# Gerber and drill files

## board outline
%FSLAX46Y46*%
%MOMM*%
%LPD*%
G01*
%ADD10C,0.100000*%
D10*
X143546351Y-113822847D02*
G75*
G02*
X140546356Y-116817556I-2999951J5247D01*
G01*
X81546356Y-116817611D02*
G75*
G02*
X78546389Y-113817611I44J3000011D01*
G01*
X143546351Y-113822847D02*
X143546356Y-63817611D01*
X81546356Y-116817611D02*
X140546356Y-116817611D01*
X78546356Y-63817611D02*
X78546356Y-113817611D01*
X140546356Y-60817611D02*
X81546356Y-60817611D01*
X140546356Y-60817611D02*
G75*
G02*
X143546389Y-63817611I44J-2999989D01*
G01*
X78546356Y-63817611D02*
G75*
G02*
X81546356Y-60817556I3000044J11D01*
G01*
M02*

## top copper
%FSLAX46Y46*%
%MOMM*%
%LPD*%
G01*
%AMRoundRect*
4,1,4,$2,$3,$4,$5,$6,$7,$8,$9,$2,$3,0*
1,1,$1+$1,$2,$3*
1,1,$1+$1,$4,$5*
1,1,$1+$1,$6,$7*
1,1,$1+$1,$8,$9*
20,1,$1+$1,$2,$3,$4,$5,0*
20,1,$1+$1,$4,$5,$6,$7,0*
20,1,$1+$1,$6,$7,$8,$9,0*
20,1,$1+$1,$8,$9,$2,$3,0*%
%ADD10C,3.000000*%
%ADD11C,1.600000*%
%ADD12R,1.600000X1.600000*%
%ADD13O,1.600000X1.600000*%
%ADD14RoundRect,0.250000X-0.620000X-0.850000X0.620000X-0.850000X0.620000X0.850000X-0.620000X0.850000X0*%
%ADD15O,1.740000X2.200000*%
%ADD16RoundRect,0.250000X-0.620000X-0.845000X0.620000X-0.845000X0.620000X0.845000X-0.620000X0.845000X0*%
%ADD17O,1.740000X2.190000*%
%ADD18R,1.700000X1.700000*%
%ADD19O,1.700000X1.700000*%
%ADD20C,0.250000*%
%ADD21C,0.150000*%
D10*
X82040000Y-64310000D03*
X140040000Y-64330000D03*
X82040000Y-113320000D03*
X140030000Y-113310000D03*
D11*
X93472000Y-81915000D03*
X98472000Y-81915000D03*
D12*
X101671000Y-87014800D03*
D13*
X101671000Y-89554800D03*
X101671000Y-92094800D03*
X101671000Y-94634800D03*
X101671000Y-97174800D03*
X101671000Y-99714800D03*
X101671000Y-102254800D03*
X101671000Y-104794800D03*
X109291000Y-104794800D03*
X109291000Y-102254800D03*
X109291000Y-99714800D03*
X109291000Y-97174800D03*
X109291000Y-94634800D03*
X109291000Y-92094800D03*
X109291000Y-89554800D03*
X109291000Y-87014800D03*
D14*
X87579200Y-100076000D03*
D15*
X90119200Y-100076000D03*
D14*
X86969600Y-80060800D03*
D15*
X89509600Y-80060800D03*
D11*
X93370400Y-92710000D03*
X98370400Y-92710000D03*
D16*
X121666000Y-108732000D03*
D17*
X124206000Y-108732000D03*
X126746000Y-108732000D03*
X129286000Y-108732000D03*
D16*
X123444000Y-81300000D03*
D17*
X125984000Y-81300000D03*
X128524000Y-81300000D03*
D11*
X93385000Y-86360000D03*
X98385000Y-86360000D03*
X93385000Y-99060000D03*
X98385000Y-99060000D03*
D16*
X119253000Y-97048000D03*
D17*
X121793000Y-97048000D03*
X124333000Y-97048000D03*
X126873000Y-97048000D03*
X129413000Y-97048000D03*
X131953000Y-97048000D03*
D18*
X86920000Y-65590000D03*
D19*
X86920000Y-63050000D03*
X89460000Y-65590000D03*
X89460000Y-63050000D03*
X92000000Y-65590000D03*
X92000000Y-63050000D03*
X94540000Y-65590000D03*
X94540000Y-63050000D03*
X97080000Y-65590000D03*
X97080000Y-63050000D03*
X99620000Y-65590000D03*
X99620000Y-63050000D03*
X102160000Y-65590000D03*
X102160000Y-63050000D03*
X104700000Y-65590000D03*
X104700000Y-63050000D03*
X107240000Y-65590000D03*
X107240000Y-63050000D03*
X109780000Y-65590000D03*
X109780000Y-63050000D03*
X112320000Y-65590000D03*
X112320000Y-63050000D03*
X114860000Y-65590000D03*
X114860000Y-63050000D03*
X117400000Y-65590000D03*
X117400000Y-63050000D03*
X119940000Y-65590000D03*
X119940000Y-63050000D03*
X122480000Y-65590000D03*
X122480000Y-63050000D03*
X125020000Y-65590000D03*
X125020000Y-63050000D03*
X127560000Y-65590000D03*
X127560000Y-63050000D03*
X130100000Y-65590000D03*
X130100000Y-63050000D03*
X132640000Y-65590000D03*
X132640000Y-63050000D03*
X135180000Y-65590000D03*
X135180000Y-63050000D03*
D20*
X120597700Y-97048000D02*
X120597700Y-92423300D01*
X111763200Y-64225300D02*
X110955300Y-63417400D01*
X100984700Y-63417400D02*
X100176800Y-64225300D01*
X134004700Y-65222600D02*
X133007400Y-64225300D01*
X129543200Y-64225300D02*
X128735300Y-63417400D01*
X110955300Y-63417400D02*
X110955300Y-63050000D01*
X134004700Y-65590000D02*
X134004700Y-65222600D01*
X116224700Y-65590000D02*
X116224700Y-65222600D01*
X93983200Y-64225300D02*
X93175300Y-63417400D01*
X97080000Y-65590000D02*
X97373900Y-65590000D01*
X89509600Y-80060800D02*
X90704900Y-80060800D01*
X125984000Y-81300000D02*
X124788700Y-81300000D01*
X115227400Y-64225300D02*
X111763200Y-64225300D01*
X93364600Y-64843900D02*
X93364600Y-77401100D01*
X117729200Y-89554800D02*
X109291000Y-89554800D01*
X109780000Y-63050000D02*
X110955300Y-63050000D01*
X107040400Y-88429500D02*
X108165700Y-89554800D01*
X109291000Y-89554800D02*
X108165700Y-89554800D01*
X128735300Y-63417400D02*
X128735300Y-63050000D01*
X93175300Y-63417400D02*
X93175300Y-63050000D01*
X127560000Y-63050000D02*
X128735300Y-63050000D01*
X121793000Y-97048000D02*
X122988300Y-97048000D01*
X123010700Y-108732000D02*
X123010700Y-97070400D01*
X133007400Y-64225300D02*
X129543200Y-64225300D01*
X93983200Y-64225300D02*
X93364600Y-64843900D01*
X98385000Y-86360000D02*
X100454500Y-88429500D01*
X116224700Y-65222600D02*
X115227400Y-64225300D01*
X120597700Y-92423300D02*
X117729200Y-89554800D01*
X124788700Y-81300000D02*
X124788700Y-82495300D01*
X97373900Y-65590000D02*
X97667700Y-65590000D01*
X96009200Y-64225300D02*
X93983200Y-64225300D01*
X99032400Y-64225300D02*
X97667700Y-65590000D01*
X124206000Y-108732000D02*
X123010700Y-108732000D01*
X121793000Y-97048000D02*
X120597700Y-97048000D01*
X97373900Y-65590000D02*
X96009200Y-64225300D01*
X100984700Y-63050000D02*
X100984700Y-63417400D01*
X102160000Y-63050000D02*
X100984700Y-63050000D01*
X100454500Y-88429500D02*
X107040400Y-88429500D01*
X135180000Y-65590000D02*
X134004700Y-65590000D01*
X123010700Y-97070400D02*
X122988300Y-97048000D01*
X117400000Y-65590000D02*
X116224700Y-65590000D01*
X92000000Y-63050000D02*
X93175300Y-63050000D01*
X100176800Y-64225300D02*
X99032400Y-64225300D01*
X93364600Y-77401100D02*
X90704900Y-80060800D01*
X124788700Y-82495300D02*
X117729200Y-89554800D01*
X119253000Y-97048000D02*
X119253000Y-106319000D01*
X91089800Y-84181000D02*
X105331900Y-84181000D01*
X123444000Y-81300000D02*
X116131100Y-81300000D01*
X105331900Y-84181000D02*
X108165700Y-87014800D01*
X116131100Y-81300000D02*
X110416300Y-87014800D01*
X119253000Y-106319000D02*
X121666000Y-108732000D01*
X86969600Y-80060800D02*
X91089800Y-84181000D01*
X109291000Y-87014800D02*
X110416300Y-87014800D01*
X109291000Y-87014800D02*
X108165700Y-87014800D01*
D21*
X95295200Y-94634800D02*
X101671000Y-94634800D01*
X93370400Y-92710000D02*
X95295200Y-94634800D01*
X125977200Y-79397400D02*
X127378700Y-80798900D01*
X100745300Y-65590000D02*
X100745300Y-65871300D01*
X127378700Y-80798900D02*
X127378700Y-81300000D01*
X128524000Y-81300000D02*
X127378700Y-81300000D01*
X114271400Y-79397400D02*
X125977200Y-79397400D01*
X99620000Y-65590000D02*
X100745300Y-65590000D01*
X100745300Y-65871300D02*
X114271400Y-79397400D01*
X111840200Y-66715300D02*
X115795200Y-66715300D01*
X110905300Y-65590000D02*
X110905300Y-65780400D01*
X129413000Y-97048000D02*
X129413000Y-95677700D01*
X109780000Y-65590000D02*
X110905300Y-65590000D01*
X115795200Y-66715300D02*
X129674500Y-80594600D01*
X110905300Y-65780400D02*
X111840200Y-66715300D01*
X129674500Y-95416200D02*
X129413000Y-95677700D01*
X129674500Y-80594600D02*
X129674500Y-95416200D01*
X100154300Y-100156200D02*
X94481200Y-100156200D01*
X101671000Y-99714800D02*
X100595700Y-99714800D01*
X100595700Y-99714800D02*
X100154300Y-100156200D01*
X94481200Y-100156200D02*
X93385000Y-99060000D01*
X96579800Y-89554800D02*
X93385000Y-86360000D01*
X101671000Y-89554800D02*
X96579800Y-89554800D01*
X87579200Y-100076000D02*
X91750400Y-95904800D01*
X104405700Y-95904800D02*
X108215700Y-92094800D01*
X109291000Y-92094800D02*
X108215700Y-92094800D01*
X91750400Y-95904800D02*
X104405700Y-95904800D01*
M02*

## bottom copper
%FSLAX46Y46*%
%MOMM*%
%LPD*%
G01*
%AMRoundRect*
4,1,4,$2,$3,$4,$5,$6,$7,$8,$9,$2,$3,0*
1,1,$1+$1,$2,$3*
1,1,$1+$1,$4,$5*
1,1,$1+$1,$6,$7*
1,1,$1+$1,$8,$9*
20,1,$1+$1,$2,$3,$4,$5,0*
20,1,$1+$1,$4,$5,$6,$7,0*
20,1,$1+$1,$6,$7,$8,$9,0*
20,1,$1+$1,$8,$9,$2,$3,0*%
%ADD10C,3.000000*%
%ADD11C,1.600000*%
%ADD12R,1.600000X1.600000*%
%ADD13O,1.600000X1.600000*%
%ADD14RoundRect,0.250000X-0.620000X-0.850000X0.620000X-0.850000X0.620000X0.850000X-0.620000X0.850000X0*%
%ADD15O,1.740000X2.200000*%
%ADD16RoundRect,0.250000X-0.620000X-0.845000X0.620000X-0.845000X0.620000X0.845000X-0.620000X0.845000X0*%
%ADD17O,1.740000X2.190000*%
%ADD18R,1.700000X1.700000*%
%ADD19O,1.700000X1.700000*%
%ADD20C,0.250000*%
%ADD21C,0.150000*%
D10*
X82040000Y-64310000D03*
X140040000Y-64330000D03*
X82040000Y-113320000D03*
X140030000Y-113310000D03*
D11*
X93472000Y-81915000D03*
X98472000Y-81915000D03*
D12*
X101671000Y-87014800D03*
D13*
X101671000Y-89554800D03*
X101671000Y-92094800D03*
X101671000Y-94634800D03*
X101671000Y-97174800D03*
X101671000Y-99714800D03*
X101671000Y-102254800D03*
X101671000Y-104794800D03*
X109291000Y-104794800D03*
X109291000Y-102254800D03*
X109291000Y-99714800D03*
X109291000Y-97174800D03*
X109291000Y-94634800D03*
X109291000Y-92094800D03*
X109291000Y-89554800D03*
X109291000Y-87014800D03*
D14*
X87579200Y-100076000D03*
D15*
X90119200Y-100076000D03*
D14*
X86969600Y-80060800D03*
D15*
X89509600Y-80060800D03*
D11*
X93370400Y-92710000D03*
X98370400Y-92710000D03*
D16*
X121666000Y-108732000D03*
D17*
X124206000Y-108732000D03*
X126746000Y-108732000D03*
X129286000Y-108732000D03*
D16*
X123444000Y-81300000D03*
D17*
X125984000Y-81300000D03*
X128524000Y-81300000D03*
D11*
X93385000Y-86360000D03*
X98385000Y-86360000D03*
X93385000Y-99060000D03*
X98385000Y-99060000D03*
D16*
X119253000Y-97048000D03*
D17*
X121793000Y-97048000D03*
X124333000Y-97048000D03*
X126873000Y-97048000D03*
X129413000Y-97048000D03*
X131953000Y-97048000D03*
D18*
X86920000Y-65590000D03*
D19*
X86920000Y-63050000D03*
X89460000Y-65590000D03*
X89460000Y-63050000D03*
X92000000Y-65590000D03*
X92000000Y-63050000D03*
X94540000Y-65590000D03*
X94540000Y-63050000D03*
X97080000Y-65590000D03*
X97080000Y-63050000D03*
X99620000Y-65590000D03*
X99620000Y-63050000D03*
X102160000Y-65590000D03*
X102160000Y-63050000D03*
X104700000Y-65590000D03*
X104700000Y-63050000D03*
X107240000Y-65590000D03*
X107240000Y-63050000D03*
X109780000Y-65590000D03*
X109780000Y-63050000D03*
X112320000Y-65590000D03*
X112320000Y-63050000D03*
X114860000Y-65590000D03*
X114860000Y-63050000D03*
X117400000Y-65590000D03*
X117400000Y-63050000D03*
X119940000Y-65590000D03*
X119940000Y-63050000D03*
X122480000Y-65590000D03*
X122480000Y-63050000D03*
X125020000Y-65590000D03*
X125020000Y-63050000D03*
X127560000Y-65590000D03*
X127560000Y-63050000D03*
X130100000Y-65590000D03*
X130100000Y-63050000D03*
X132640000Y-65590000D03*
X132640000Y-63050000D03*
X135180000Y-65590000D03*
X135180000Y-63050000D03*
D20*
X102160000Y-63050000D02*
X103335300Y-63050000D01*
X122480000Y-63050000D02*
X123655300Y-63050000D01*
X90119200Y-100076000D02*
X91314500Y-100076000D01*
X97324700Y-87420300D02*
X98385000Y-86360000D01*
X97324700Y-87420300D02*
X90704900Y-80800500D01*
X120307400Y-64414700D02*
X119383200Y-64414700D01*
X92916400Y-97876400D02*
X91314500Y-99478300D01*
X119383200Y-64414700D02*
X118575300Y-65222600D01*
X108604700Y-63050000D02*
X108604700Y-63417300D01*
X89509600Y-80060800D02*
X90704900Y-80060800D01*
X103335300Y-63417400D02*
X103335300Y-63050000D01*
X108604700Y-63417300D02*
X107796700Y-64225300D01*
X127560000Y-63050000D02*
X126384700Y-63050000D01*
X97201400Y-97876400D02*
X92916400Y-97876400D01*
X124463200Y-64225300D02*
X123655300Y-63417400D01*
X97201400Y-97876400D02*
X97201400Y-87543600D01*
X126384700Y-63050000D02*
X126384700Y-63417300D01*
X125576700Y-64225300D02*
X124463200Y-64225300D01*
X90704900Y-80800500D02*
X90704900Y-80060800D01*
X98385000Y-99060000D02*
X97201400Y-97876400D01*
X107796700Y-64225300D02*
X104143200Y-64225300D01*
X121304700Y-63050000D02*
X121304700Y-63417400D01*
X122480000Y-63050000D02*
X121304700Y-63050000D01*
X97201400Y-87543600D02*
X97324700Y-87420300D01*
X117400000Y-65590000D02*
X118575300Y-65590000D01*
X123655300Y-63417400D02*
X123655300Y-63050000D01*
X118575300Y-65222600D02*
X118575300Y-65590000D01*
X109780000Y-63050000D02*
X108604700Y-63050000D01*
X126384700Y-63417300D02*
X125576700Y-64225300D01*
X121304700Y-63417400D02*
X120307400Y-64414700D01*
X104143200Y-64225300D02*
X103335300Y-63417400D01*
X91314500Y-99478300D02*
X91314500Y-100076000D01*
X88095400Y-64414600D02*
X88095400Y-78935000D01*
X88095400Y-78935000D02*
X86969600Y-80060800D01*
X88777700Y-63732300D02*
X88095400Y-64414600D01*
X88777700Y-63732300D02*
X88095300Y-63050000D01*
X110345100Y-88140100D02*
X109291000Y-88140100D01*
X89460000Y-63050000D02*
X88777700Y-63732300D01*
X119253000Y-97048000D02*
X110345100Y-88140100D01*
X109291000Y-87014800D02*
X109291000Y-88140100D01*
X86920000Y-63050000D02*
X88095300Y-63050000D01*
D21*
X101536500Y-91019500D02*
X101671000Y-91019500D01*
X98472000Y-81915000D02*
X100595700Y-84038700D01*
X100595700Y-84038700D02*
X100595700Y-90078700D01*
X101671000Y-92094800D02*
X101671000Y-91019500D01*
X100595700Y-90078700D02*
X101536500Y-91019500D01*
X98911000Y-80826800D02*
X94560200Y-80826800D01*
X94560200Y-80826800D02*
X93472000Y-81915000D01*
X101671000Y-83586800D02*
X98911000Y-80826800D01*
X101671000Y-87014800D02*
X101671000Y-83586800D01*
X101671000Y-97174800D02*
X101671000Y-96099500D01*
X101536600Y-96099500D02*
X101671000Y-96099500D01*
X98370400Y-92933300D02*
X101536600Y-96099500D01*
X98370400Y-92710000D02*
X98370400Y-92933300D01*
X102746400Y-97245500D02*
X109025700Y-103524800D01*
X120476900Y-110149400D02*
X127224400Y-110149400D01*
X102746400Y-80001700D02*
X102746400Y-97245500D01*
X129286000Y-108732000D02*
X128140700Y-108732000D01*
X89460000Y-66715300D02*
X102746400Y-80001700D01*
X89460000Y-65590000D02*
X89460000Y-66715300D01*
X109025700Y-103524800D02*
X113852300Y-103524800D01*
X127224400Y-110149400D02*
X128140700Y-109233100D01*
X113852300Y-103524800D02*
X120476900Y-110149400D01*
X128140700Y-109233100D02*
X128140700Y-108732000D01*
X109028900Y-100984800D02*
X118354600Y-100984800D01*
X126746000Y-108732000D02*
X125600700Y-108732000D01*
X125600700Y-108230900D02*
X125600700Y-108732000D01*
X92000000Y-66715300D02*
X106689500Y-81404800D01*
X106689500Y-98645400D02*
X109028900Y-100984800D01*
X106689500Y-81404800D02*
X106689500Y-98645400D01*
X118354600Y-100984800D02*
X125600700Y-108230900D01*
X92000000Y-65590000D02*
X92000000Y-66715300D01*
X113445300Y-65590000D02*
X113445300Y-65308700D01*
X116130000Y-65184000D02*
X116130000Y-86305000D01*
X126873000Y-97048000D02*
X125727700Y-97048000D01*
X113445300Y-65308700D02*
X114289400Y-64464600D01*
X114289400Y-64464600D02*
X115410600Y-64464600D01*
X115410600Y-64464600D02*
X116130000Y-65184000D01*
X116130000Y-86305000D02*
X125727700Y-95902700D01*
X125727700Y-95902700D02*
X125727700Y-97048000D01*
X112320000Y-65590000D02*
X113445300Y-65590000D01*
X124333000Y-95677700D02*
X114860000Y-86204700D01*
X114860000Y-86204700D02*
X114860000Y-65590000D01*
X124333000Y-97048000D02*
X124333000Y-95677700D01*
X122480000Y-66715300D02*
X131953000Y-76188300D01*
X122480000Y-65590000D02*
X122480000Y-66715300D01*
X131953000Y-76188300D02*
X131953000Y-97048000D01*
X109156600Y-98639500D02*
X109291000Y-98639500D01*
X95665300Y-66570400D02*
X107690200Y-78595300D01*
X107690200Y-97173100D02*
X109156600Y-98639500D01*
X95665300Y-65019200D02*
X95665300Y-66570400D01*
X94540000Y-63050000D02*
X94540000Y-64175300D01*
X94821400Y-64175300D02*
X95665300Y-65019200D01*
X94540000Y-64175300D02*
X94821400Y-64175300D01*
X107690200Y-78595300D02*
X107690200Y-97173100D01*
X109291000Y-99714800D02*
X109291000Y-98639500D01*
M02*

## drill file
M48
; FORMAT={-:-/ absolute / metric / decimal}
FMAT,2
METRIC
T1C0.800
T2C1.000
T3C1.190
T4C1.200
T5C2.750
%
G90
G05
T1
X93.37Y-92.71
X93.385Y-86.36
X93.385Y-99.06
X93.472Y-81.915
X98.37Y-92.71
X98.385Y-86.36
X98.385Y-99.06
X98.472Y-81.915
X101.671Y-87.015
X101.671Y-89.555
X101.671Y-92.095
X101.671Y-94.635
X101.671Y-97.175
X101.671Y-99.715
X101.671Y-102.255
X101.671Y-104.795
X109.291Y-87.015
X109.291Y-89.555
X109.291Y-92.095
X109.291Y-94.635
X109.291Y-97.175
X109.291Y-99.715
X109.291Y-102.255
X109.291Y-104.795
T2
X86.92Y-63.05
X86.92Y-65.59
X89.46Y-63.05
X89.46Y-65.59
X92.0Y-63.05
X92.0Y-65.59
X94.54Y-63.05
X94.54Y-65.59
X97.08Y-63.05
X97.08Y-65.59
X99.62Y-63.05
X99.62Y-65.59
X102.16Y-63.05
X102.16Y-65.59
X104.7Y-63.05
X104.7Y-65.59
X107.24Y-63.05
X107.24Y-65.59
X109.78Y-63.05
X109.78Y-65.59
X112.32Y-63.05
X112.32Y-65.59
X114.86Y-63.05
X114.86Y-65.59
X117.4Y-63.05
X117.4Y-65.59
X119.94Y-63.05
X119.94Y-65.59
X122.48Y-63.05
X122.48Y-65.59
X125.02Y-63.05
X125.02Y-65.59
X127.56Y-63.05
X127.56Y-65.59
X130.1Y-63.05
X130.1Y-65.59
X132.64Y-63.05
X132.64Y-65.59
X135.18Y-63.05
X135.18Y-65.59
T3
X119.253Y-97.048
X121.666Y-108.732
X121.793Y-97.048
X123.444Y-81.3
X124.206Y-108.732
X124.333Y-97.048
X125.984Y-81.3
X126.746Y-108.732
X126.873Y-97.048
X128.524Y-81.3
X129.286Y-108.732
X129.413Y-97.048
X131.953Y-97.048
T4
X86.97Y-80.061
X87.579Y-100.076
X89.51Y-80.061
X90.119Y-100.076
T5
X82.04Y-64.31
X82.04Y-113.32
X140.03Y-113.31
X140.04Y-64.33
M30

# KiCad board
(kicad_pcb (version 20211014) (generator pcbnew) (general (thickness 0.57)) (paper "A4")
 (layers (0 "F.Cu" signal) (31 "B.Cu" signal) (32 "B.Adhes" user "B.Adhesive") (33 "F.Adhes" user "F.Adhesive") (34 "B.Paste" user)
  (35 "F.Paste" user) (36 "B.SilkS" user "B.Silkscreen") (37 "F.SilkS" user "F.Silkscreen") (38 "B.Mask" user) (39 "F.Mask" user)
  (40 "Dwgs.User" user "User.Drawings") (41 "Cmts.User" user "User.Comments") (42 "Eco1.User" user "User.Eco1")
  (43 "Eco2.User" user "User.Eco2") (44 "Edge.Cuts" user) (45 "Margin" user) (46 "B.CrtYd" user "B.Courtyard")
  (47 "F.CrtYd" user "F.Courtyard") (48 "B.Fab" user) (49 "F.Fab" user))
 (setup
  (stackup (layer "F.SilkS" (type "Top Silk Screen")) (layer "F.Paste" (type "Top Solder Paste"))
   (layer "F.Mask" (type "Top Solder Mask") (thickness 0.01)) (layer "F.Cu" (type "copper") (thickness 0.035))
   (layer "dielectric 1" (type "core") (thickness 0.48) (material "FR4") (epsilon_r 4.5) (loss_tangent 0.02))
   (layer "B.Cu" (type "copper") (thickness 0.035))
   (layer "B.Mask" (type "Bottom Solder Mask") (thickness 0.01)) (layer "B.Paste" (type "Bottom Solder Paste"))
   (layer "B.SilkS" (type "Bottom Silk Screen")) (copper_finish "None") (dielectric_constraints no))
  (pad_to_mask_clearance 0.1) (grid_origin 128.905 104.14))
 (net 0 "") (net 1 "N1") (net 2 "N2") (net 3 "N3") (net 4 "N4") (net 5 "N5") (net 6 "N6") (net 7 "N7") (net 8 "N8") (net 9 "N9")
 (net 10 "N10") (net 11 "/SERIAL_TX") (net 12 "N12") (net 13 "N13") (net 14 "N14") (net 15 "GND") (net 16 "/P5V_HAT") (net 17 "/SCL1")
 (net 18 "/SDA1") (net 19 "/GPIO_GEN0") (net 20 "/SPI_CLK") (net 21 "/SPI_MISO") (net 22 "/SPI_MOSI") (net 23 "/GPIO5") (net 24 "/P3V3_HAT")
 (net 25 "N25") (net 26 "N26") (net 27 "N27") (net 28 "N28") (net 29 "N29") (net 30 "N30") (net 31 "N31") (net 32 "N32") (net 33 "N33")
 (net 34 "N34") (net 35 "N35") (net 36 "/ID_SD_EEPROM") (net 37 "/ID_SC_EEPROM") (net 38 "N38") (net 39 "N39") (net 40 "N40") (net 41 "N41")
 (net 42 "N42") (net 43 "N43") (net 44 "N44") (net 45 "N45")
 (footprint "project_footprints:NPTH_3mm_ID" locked (layer "F.Cu") (at 82.04 64.31)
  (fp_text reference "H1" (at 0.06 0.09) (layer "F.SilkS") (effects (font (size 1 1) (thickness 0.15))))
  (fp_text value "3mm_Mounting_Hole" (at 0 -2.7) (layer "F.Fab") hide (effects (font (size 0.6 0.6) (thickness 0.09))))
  (pad "" np_thru_hole circle locked (at 0 0) (size 3 3) (drill 2.75) (layers *.Cu *.Mask) (clearance 1.6)))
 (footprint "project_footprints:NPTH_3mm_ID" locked (layer "F.Cu") (at 140.04 64.33)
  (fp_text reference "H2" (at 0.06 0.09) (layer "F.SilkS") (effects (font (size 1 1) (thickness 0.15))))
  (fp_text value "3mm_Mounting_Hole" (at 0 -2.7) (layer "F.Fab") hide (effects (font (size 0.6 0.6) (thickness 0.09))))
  (pad "" np_thru_hole circle locked (at 0 0) (size 3 3) (drill 2.75) (layers *.Cu *.Mask) (clearance 1.6)))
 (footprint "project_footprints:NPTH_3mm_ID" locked (layer "F.Cu") (at 82.04 113.32)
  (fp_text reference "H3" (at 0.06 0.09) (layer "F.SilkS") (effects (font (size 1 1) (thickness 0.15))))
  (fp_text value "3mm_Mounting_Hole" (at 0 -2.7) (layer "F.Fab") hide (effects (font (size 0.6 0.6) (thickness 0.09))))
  (pad "" np_thru_hole circle locked (at 0 0) (size 3 3) (drill 2.75) (layers *.Cu *.Mask) (clearance 1.6)))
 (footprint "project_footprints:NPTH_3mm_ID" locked (layer "F.Cu") (at 140.03 113.31)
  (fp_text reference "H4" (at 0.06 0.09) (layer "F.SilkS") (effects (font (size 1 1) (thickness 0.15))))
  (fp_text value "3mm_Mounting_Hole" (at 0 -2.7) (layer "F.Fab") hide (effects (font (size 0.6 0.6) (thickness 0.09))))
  (pad "" np_thru_hole circle locked (at 0 0) (size 3 3) (drill 2.75) (layers *.Cu *.Mask) (clearance 1.6)))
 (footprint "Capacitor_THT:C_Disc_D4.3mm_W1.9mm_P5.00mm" (layer "F.Cu") (at 93.472 81.915)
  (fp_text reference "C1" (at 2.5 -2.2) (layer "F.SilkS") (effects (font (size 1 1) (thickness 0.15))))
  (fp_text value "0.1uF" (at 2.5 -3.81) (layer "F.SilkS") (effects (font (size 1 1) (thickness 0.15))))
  (pad "1" thru_hole circle locked (at 0 0) (size 1.6 1.6) (drill 0.8) (layers *.Cu *.Mask) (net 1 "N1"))
  (pad "2" thru_hole circle locked (at 5 0) (size 1.6 1.6) (drill 0.8) (layers *.Cu *.Mask) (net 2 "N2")))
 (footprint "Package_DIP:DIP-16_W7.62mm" (layer "F.Cu") (at 101.671 87.0148)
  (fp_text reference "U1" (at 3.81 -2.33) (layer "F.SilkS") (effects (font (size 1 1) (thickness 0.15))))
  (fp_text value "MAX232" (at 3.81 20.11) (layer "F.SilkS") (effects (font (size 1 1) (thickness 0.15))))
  (pad "1" thru_hole rect locked (at 0 0) (size 1.6 1.6) (drill 0.8) (layers *.Cu *.Mask) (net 1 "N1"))
  (pad "2" thru_hole oval locked (at 0 2.54) (size 1.6 1.6) (drill 0.8) (layers *.Cu *.Mask) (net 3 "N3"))
  (pad "3" thru_hole oval locked (at 0 5.08) (size 1.6 1.6) (drill 0.8) (layers *.Cu *.Mask) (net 2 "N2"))
  (pad "4" thru_hole oval locked (at 0 7.62) (size 1.6 1.6) (drill 0.8) (layers *.Cu *.Mask) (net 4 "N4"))
  (pad "5" thru_hole oval locked (at 0 10.16) (size 1.6 1.6) (drill 0.8) (layers *.Cu *.Mask) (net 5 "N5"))
  (pad "6" thru_hole oval locked (at 0 12.7) (size 1.6 1.6) (drill 0.8) (layers *.Cu *.Mask) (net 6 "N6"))
  (pad "7" thru_hole oval locked (at 0 15.24) (size 1.6 1.6) (drill 0.8) (layers *.Cu *.Mask) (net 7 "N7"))
  (pad "8" thru_hole oval locked (at 0 17.78) (size 1.6 1.6) (drill 0.8) (layers *.Cu *.Mask) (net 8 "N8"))
  (pad "9" thru_hole oval locked (at 7.62 17.78) (size 1.6 1.6) (drill 0.8) (layers *.Cu *.Mask) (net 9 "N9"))
  (pad "10" thru_hole oval locked (at 7.62 15.24) (size 1.6 1.6) (drill 0.8) (layers *.Cu *.Mask) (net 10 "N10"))
  (pad "11" thru_hole oval locked (at 7.62 12.7) (size 1.6 1.6) (drill 0.8) (layers *.Cu *.Mask) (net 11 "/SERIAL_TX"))
  (pad "12" thru_hole oval locked (at 7.62 10.16) (size 1.6 1.6) (drill 0.8) (layers *.Cu *.Mask) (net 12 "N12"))
  (pad "13" thru_hole oval locked (at 7.62 7.62) (size 1.6 1.6) (drill 0.8) (layers *.Cu *.Mask) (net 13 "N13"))
  (pad "14" thru_hole oval locked (at 7.62 5.08) (size 1.6 1.6) (drill 0.8) (layers *.Cu *.Mask) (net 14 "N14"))
  (pad "15" thru_hole oval locked (at 7.62 2.54) (size 1.6 1.6) (drill 0.8) (layers *.Cu *.Mask) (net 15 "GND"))
  (pad "16" thru_hole oval locked (at 7.62 0) (size 1.6 1.6) (drill 0.8) (layers *.Cu *.Mask) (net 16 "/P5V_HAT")))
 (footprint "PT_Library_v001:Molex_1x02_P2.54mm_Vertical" (layer "F.Cu") (at 87.5792 100.076)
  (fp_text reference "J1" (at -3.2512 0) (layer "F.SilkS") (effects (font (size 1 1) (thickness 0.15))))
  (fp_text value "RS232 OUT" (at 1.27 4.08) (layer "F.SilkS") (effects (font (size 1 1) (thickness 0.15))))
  (pad "1" thru_hole roundrect locked (at 0 0) (size 1.74 2.2) (drill 1.2) (layers *.Cu *.Mask) (roundrect_rratio 0.1436781609)
   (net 14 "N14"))
  (pad "2" thru_hole oval locked (at 2.54 0) (size 1.74 2.2) (drill 1.2) (layers *.Cu *.Mask) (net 15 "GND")))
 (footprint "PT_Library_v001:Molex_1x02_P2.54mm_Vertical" (layer "F.Cu") (at 86.9696 80.0608)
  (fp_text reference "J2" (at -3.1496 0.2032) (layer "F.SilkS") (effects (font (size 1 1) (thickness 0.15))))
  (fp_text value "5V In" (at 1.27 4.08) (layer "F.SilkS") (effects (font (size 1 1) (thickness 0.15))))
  (pad "1" thru_hole roundrect locked (at 0 0) (size 1.74 2.2) (drill 1.2) (layers *.Cu *.Mask) (roundrect_rratio 0.1436781609)
   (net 16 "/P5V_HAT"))
  (pad "2" thru_hole oval locked (at 2.54 0) (size 1.74 2.2) (drill 1.2) (layers *.Cu *.Mask) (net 15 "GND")))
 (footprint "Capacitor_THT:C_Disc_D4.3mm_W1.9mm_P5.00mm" (layer "F.Cu") (at 93.3704 92.71)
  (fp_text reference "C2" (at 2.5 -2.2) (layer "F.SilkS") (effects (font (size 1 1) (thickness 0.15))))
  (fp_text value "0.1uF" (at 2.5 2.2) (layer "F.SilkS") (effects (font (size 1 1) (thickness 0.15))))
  (pad "1" thru_hole circle locked (at 0 0) (size 1.6 1.6) (drill 0.8) (layers *.Cu *.Mask) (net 4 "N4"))
  (pad "2" thru_hole circle locked (at 5 0) (size 1.6 1.6) (drill 0.8) (layers *.Cu *.Mask) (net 5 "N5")))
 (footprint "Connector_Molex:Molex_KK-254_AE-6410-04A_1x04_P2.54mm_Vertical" (layer "F.Cu") (at 121.666 108.732)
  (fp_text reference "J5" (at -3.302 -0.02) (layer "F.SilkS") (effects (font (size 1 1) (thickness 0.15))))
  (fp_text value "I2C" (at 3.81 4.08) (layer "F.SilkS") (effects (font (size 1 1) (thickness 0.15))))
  (pad "1" thru_hole roundrect (at 0 0) (size 1.74 2.19) (drill 1.19) (layers *.Cu *.Mask) (roundrect_rratio 0.1436781609)
   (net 16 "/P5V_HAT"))
  (pad "2" thru_hole oval (at 2.54 0) (size 1.74 2.19) (drill 1.19) (layers *.Cu *.Mask) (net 15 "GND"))
  (pad "3" thru_hole oval (at 5.08 0) (size 1.74 2.19) (drill 1.19) (layers *.Cu *.Mask) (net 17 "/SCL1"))
  (pad "4" thru_hole oval (at 7.62 0) (size 1.74 2.19) (drill 1.19) (layers *.Cu *.Mask) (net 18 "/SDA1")))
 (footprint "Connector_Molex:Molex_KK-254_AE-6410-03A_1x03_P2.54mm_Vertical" (layer "F.Cu") (at 123.444 81.3)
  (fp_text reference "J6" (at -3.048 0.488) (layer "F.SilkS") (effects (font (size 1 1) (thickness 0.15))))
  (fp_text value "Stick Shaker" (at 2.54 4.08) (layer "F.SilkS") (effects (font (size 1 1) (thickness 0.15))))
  (pad "1" thru_hole roundrect (at 0 0) (size 1.74 2.19) (drill 1.19) (layers *.Cu *.Mask) (roundrect_rratio 0.1436781609)
   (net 16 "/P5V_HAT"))
  (pad "2" thru_hole oval (at 2.54 0) (size 1.74 2.19) (drill 1.19) (layers *.Cu *.Mask) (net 15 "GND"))
  (pad "3" thru_hole oval (at 5.08 0) (size 1.74 2.19) (drill 1.19) (layers *.Cu *.Mask) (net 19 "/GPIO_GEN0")))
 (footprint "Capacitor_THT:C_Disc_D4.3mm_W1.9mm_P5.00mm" (layer "F.Cu") (at 93.385 86.36)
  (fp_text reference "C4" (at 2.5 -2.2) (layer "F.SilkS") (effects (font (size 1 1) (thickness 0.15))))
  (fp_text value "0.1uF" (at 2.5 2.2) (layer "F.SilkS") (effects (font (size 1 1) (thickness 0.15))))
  (pad "1" thru_hole circle (at 0 0) (size 1.6 1.6) (drill 0.8) (layers *.Cu *.Mask) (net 3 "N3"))
  (pad "2" thru_hole circle (at 5 0) (size 1.6 1.6) (drill 0.8) (layers *.Cu *.Mask) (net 15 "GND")))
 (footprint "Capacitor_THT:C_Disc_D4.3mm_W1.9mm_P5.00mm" (layer "F.Cu") (at 93.385 99.06)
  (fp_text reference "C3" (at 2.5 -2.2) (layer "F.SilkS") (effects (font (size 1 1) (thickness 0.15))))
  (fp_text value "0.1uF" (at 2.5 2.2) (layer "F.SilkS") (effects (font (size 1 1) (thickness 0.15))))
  (pad "1" thru_hole circle (at 0 0) (size 1.6 1.6) (drill 0.8) (layers *.Cu *.Mask) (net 6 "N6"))
  (pad "2" thru_hole circle (at 5 0) (size 1.6 1.6) (drill 0.8) (layers *.Cu *.Mask) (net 15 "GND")))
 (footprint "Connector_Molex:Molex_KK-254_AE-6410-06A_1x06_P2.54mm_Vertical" (layer "F.Cu") (at 119.253 97.048)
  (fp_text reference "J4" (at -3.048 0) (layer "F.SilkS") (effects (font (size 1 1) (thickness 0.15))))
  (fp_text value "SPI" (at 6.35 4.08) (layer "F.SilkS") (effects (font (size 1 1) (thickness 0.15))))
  (pad "1" thru_hole roundrect (at 0 0) (size 1.74 2.19) (drill 1.19) (layers *.Cu *.Mask) (roundrect_rratio 0.1436781609)
   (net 16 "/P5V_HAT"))
  (pad "2" thru_hole oval (at 2.54 0) (size 1.74 2.19) (drill 1.19) (layers *.Cu *.Mask) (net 15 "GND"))
  (pad "3" thru_hole oval (at 5.08 0) (size 1.74 2.19) (drill 1.19) (layers *.Cu *.Mask) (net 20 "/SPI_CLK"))
  (pad "4" thru_hole oval (at 7.62 0) (size 1.74 2.19) (drill 1.19) (layers *.Cu *.Mask) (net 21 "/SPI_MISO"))
  (pad "5" thru_hole oval (at 10.16 0) (size 1.74 2.19) (drill 1.19) (layers *.Cu *.Mask) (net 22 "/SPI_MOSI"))
  (pad "6" thru_hole oval (at 12.7 0) (size 1.74 2.19) (drill 1.19) (layers *.Cu *.Mask) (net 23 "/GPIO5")))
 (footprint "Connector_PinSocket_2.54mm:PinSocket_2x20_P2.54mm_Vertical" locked (layer "B.Cu") (at 86.92 65.59 -90)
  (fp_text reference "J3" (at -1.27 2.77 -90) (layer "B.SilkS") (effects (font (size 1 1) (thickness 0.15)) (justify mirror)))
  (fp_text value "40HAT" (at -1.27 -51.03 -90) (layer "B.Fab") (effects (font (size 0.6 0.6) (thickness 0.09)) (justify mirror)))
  (pad "1" thru_hole rect locked (at 0 0 270) (size 1.7 1.7) (drill 1) (layers *.Cu *.Mask) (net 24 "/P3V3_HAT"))
  (pad "2" thru_hole oval locked (at -2.54 0 270) (size 1.7 1.7) (drill 1) (layers *.Cu *.Mask) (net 16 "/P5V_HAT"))
  (pad "3" thru_hole oval locked (at 0 -2.54 270) (size 1.7 1.7) (drill 1) (layers *.Cu *.Mask) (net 18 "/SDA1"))
  (pad "4" thru_hole oval locked (at -2.54 -2.54 270) (size 1.7 1.7) (drill 1) (layers *.Cu *.Mask) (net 16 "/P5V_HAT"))
  (pad "5" thru_hole oval locked (at 0 -5.08 270) (size 1.7 1.7) (drill 1) (layers *.Cu *.Mask) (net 17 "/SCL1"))
  (pad "6" thru_hole oval locked (at -2.54 -5.08 270) (size 1.7 1.7) (drill 1) (layers *.Cu *.Mask) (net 15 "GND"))
  (pad "7" thru_hole oval locked (at 0 -7.62 270) (size 1.7 1.7) (drill 1) (layers *.Cu *.Mask) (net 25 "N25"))
  (pad "8" thru_hole oval locked (at -2.54 -7.62 270) (size 1.7 1.7) (drill 1) (layers *.Cu *.Mask) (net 11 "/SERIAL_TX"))
  (pad "9" thru_hole oval locked (at 0 -10.16 270) (size 1.7 1.7) (drill 1) (layers *.Cu *.Mask) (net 15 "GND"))
  (pad "10" thru_hole oval locked (at -2.54 -10.16 270) (size 1.7 1.7) (drill 1) (layers *.Cu *.Mask) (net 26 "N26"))
  (pad "11" thru_hole oval locked (at 0 -12.7 270) (size 1.7 1.7) (drill 1) (layers *.Cu *.Mask) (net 19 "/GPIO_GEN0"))
  (pad "12" thru_hole oval locked (at -2.54 -12.7 270) (size 1.7 1.7) (drill 1) (layers *.Cu *.Mask) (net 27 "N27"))
  (pad "13" thru_hole oval locked (at 0 -15.24 270) (size 1.7 1.7) (drill 1) (layers *.Cu *.Mask) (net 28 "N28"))
  (pad "14" thru_hole oval locked (at -2.54 -15.24 270) (size 1.7 1.7) (drill 1) (layers *.Cu *.Mask) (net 15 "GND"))
  (pad "15" thru_hole oval locked (at 0 -17.78 270) (size 1.7 1.7) (drill 1) (layers *.Cu *.Mask) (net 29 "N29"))
  (pad "16" thru_hole oval locked (at -2.54 -17.78 270) (size 1.7 1.7) (drill 1) (layers *.Cu *.Mask) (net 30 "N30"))
  (pad "17" thru_hole oval locked (at 0 -20.32 270) (size 1.7 1.7) (drill 1) (layers *.Cu *.Mask) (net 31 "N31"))
  (pad "18" thru_hole oval locked (at -2.54 -20.32 270) (size 1.7 1.7) (drill 1) (layers *.Cu *.Mask) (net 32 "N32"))
  (pad "19" thru_hole oval locked (at 0 -22.86 270) (size 1.7 1.7) (drill 1) (layers *.Cu *.Mask) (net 22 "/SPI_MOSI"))
  (pad "20" thru_hole oval locked (at -2.54 -22.86 270) (size 1.7 1.7) (drill 1) (layers *.Cu *.Mask) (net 15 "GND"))
  (pad "21" thru_hole oval locked (at 0 -25.4 270) (size 1.7 1.7) (drill 1) (layers *.Cu *.Mask) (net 21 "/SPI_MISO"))
  (pad "22" thru_hole oval locked (at -2.54 -25.4 270) (size 1.7 1.7) (drill 1) (layers *.Cu *.Mask) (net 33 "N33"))
  (pad "23" thru_hole oval locked (at 0 -27.94 270) (size 1.7 1.7) (drill 1) (layers *.Cu *.Mask) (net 20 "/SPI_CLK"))
  (pad "24" thru_hole oval locked (at -2.54 -27.94 270) (size 1.7 1.7) (drill 1) (layers *.Cu *.Mask) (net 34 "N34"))
  (pad "25" thru_hole oval locked (at 0 -30.48 270) (size 1.7 1.7) (drill 1) (layers *.Cu *.Mask) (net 15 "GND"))
  (pad "26" thru_hole oval locked (at -2.54 -30.48 270) (size 1.7 1.7) (drill 1) (layers *.Cu *.Mask) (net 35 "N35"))
  (pad "27" thru_hole oval locked (at 0 -33.02 270) (size 1.7 1.7) (drill 1) (layers *.Cu *.Mask) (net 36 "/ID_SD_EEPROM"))
  (pad "28" thru_hole oval locked (at -2.54 -33.02 270) (size 1.7 1.7) (drill 1) (layers *.Cu *.Mask) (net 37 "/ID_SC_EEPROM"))
  (pad "29" thru_hole oval locked (at 0 -35.56 270) (size 1.7 1.7) (drill 1) (layers *.Cu *.Mask) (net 23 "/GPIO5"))
  (pad "30" thru_hole oval locked (at -2.54 -35.56 270) (size 1.7 1.7) (drill 1) (layers *.Cu *.Mask) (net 15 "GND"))
  (pad "31" thru_hole oval locked (at 0 -38.1 270) (size 1.7 1.7) (drill 1) (layers *.Cu *.Mask) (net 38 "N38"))
  (pad "32" thru_hole oval locked (at -2.54 -38.1 270) (size 1.7 1.7) (drill 1) (layers *.Cu *.Mask) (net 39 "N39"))
  (pad "33" thru_hole oval locked (at 0 -40.64 270) (size 1.7 1.7) (drill 1) (layers *.Cu *.Mask) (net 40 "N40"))
  (pad "34" thru_hole oval locked (at -2.54 -40.64 270) (size 1.7 1.7) (drill 1) (layers *.Cu *.Mask) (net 15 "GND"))
  (pad "35" thru_hole oval locked (at 0 -43.18 270) (size 1.7 1.7) (drill 1) (layers *.Cu *.Mask) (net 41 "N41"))
  (pad "36" thru_hole oval locked (at -2.54 -43.18 270) (size 1.7 1.7) (drill 1) (layers *.Cu *.Mask) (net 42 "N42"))
  (pad "37" thru_hole oval locked (at 0 -45.72 270) (size 1.7 1.7) (drill 1) (layers *.Cu *.Mask) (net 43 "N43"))
  (pad "38" thru_hole oval locked (at -2.54 -45.72 270) (size 1.7 1.7) (drill 1) (layers *.Cu *.Mask) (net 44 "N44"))
  (pad "39" thru_hole oval locked (at 0 -48.26 270) (size 1.7 1.7) (drill 1) (layers *.Cu *.Mask) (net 15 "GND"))
  (pad "40" thru_hole oval locked (at -2.54 -48.26 270) (size 1.7 1.7) (drill 1) (layers *.Cu *.Mask) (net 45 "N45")))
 (gr_arc (start 143.546351 113.822847) (mid 142.665824 115.940781) (end 140.546356 116.817611) (layer "Edge.Cuts") (width 0.1))
 (gr_arc (start 81.546356 116.817611) (mid 79.425036 115.938931) (end 78.546356 113.817611) (layer "Edge.Cuts") (width 0.1))
 (gr_line (start 143.546351 113.822847) (end 143.546356 63.817611) (layer "Edge.Cuts") (width 0.1))
 (gr_line (start 81.546356 116.817611) (end 140.546356 116.817611) (layer "Edge.Cuts") (width 0.1))
 (gr_line (start 78.546356 63.817611) (end 78.546356 113.817611) (layer "Edge.Cuts") (width 0.1))
 (gr_line (start 140.546356 60.817611) (end 81.546356 60.817611) (layer "Edge.Cuts") (width 0.1))
 (gr_arc (start 140.546356 60.817611) (mid 142.667676 61.696291) (end 143.546356 63.817611) (layer "Edge.Cuts") (width 0.1))
 (gr_arc (start 78.546356 63.817611) (mid 79.425036 61.696291) (end 81.546356 60.817611) (layer "Edge.Cuts") (width 0.1))
 (segment (start 120.5977 97.048) (end 120.5977 92.4233) (width 0.25) (layer "F.Cu") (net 15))
 (segment (start 111.7632 64.2253) (end 110.9553 63.4174) (width 0.25) (layer "F.Cu") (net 15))
 (segment (start 100.9847 63.4174) (end 100.1768 64.2253) (width 0.25) (layer "F.Cu") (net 15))
 (segment (start 134.0047 65.2226) (end 133.0074 64.2253) (width 0.25) (layer "F.Cu") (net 15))
 (segment (start 129.5432 64.2253) (end 128.7353 63.4174) (width 0.25) (layer "F.Cu") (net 15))
 (segment (start 110.9553 63.4174) (end 110.9553 63.05) (width 0.25) (layer "F.Cu") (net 15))
 (segment (start 134.0047 65.59) (end 134.0047 65.2226) (width 0.25) (layer "F.Cu") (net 15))
 (segment (start 116.2247 65.59) (end 116.2247 65.2226) (width 0.25) (layer "F.Cu") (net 15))
 (segment (start 93.9832 64.2253) (end 93.1753 63.4174) (width 0.25) (layer "F.Cu") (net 15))
 (segment (start 97.08 65.59) (end 97.3739 65.59) (width 0.25) (layer "F.Cu") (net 15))
 (segment (start 89.5096 80.0608) (end 90.7049 80.0608) (width 0.25) (layer "F.Cu") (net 15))
 (segment (start 125.984 81.3) (end 124.7887 81.3) (width 0.25) (layer "F.Cu") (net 15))
 (segment (start 115.2274 64.2253) (end 111.7632 64.2253) (width 0.25) (layer "F.Cu") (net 15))
 (segment (start 93.3646 64.8439) (end 93.3646 77.4011) (width 0.25) (layer "F.Cu") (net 15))
 (segment (start 117.7292 89.5548) (end 109.291 89.5548) (width 0.25) (layer "F.Cu") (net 15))
 (segment (start 109.78 63.05) (end 110.9553 63.05) (width 0.25) (layer "F.Cu") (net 15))
 (segment (start 107.0404 88.4295) (end 108.1657 89.5548) (width 0.25) (layer "F.Cu") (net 15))
 (segment (start 109.291 89.5548) (end 108.1657 89.5548) (width 0.25) (layer "F.Cu") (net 15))
 (segment (start 128.7353 63.4174) (end 128.7353 63.05) (width 0.25) (layer "F.Cu") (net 15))
 (segment (start 93.1753 63.4174) (end 93.1753 63.05) (width 0.25) (layer "F.Cu") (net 15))
 (segment (start 127.56 63.05) (end 128.7353 63.05) (width 0.25) (layer "F.Cu") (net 15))
 (segment (start 121.793 97.048) (end 122.9883 97.048) (width 0.25) (layer "F.Cu") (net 15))
 (segment (start 123.0107 108.732) (end 123.0107 97.0704) (width 0.25) (layer "F.Cu") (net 15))
 (segment (start 133.0074 64.2253) (end 129.5432 64.2253) (width 0.25) (layer "F.Cu") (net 15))
 (segment (start 93.9832 64.2253) (end 93.3646 64.8439) (width 0.25) (layer "F.Cu") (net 15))
 (segment (start 98.385 86.36) (end 100.4545 88.4295) (width 0.25) (layer "F.Cu") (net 15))
 (segment (start 116.2247 65.2226) (end 115.2274 64.2253) (width 0.25) (layer "F.Cu") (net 15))
 (segment (start 120.5977 92.4233) (end 117.7292 89.5548) (width 0.25) (layer "F.Cu") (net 15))
 (segment (start 124.7887 81.3) (end 124.7887 82.4953) (width 0.25) (layer "F.Cu") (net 15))
 (segment (start 97.3739 65.59) (end 97.6677 65.59) (width 0.25) (layer "F.Cu") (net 15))
 (segment (start 96.0092 64.2253) (end 93.9832 64.2253) (width 0.25) (layer "F.Cu") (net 15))
 (segment (start 99.0324 64.2253) (end 97.6677 65.59) (width 0.25) (layer "F.Cu") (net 15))
 (segment (start 124.206 108.732) (end 123.0107 108.732) (width 0.25) (layer "F.Cu") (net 15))
 (segment (start 121.793 97.048) (end 120.5977 97.048) (width 0.25) (layer "F.Cu") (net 15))
 (segment (start 97.3739 65.59) (end 96.0092 64.2253) (width 0.25) (layer "F.Cu") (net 15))
 (segment (start 100.9847 63.05) (end 100.9847 63.4174) (width 0.25) (layer "F.Cu") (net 15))
 (segment (start 102.16 63.05) (end 100.9847 63.05) (width 0.25) (layer "F.Cu") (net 15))
 (segment (start 100.4545 88.4295) (end 107.0404 88.4295) (width 0.25) (layer "F.Cu") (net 15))
 (segment (start 135.18 65.59) (end 134.0047 65.59) (width 0.25) (layer "F.Cu") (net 15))
 (segment (start 123.0107 97.0704) (end 122.9883 97.048) (width 0.25) (layer "F.Cu") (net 15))
 (segment (start 117.4 65.59) (end 116.2247 65.59) (width 0.25) (layer "F.Cu") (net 15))
 (segment (start 92 63.05) (end 93.1753 63.05) (width 0.25) (layer "F.Cu") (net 15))
 (segment (start 100.1768 64.2253) (end 99.0324 64.2253) (width 0.25) (layer "F.Cu") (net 15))
 (segment (start 93.3646 77.4011) (end 90.7049 80.0608) (width 0.25) (layer "F.Cu") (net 15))
 (segment (start 124.7887 82.4953) (end 117.7292 89.5548) (width 0.25) (layer "F.Cu") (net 15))
 (segment (start 102.16 63.05) (end 103.3353 63.05) (width 0.25) (layer "B.Cu") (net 15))
 (segment (start 122.48 63.05) (end 123.6553 63.05) (width 0.25) (layer "B.Cu") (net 15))
 (segment (start 90.1192 100.076) (end 91.3145 100.076) (width 0.25) (layer "B.Cu") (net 15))
 (segment (start 97.3247 87.4203) (end 98.385 86.36) (width 0.25) (layer "B.Cu") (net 15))
 (segment (start 97.3247 87.4203) (end 90.7049 80.8005) (width 0.25) (layer "B.Cu") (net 15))
 (segment (start 120.3074 64.4147) (end 119.3832 64.4147) (width 0.25) (layer "B.Cu") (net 15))
 (segment (start 92.9164 97.8764) (end 91.3145 99.4783) (width 0.25) (layer "B.Cu") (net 15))
 (segment (start 119.3832 64.4147) (end 118.5753 65.2226) (width 0.25) (layer "B.Cu") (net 15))
 (segment (start 108.6047 63.05) (end 108.6047 63.4173) (width 0.25) (layer "B.Cu") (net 15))
 (segment (start 89.5096 80.0608) (end 90.7049 80.0608) (width 0.25) (layer "B.Cu") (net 15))
 (segment (start 103.3353 63.4174) (end 103.3353 63.05) (width 0.25) (layer "B.Cu") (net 15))
 (segment (start 108.6047 63.4173) (end 107.7967 64.2253) (width 0.25) (layer "B.Cu") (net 15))
 (segment (start 127.56 63.05) (end 126.3847 63.05) (width 0.25) (layer "B.Cu") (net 15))
 (segment (start 97.2014 97.8764) (end 92.9164 97.8764) (width 0.25) (layer "B.Cu") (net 15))
 (segment (start 124.4632 64.2253) (end 123.6553 63.4174) (width 0.25) (layer "B.Cu") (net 15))
 (segment (start 97.2014 97.8764) (end 97.2014 87.5436) (width 0.25) (layer "B.Cu") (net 15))
 (segment (start 126.3847 63.05) (end 126.3847 63.4173) (width 0.25) (layer "B.Cu") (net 15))
 (segment (start 125.5767 64.2253) (end 124.4632 64.2253) (width 0.25) (layer "B.Cu") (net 15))
 (segment (start 90.7049 80.8005) (end 90.7049 80.0608) (width 0.25) (layer "B.Cu") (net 15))
 (segment (start 98.385 99.06) (end 97.2014 97.8764) (width 0.25) (layer "B.Cu") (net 15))
 (segment (start 107.7967 64.2253) (end 104.1432 64.2253) (width 0.25) (layer "B.Cu") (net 15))
 (segment (start 121.3047 63.05) (end 121.3047 63.4174) (width 0.25) (layer "B.Cu") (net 15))
 (segment (start 122.48 63.05) (end 121.3047 63.05) (width 0.25) (layer "B.Cu") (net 15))
 (segment (start 97.2014 87.5436) (end 97.3247 87.4203) (width 0.25) (layer "B.Cu") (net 15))
 (segment (start 117.4 65.59) (end 118.5753 65.59) (width 0.25) (layer "B.Cu") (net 15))
 (segment (start 123.6553 63.4174) (end 123.6553 63.05) (width 0.25) (layer "B.Cu") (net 15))
 (segment (start 118.5753 65.2226) (end 118.5753 65.59) (width 0.25) (layer "B.Cu") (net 15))
 (segment (start 109.78 63.05) (end 108.6047 63.05) (width 0.25) (layer "B.Cu") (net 15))
 (segment (start 126.3847 63.4173) (end 125.5767 64.2253) (width 0.25) (layer "B.Cu") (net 15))
 (segment (start 121.3047 63.4174) (end 120.3074 64.4147) (width 0.25) (layer "B.Cu") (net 15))
 (segment (start 104.1432 64.2253) (end 103.3353 63.4174) (width 0.25) (layer "B.Cu") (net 15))
 (segment (start 91.3145 99.4783) (end 91.3145 100.076) (width 0.25) (layer "B.Cu") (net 15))
 (segment (start 119.253 97.048) (end 119.253 106.319) (width 0.25) (layer "F.Cu") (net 16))
 (segment (start 91.0898 84.181) (end 105.3319 84.181) (width 0.25) (layer "F.Cu") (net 16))
 (segment (start 123.444 81.3) (end 116.1311 81.3) (width 0.25) (layer "F.Cu") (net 16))
 (segment (start 105.3319 84.181) (end 108.1657 87.0148) (width 0.25) (layer "F.Cu") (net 16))
 (segment (start 116.1311 81.3) (end 110.4163 87.0148) (width 0.25) (layer "F.Cu") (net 16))
 (segment (start 119.253 106.319) (end 121.666 108.732) (width 0.25) (layer "F.Cu") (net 16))
 (segment (start 86.9696 80.0608) (end 91.0898 84.181) (width 0.25) (layer "F.Cu") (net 16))
 (segment (start 109.291 87.0148) (end 110.4163 87.0148) (width 0.25) (layer "F.Cu") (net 16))
 (segment (start 109.291 87.0148) (end 108.1657 87.0148) (width 0.25) (layer "F.Cu") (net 16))
 (segment (start 88.0954 64.4146) (end 88.0954 78.935) (width 0.25) (layer "B.Cu") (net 16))
 (segment (start 88.0954 78.935) (end 86.9696 80.0608) (width 0.25) (layer "B.Cu") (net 16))
 (segment (start 88.7777 63.7323) (end 88.0954 64.4146) (width 0.25) (layer "B.Cu") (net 16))
 (segment (start 88.7777 63.7323) (end 88.0953 63.05) (width 0.25) (layer "B.Cu") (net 16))
 (segment (start 110.3451 88.1401) (end 109.291 88.1401) (width 0.25) (layer "B.Cu") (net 16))
 (segment (start 89.46 63.05) (end 88.7777 63.7323) (width 0.25) (layer "B.Cu") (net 16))
 (segment (start 119.253 97.048) (end 110.3451 88.1401) (width 0.25) (layer "B.Cu") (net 16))
 (segment (start 109.291 87.0148) (end 109.291 88.1401) (width 0.25) (layer "B.Cu") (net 16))
 (segment (start 86.92 63.05) (end 88.0953 63.05) (width 0.25) (layer "B.Cu") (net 16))
 (segment (start 101.5365 91.0195) (end 101.671 91.0195) (width 0.15) (layer "B.Cu") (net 2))
 (segment (start 98.472 81.915) (end 100.5957 84.0387) (width 0.15) (layer "B.Cu") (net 2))
 (segment (start 100.5957 84.0387) (end 100.5957 90.0787) (width 0.15) (layer "B.Cu") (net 2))
 (segment (start 101.671 92.0948) (end 101.671 91.0195) (width 0.15) (layer "B.Cu") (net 2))
 (segment (start 100.5957 90.0787) (end 101.5365 91.0195) (width 0.15) (layer "B.Cu") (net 2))
 (segment (start 98.911 80.8268) (end 94.5602 80.8268) (width 0.15) (layer "B.Cu") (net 1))
 (segment (start 94.5602 80.8268) (end 93.472 81.915) (width 0.15) (layer "B.Cu") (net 1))
 (segment (start 101.671 83.5868) (end 98.911 80.8268) (width 0.15) (layer "B.Cu") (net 1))
 (segment (start 101.671 87.0148) (end 101.671 83.5868) (width 0.15) (layer "B.Cu") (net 1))
 (segment (start 101.671 97.1748) (end 101.671 96.0995) (width 0.15) (layer "B.Cu") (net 5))
 (segment (start 101.5366 96.0995) (end 101.671 96.0995) (width 0.15) (layer "B.Cu") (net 5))
 (segment (start 98.3704 92.9333) (end 101.5366 96.0995) (width 0.15) (layer "B.Cu") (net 5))
 (segment (start 98.3704 92.71) (end 98.3704 92.9333) (width 0.15) (layer "B.Cu") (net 5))
 (segment (start 95.2952 94.6348) (end 101.671 94.6348) (width 0.15) (layer "F.Cu") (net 4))
 (segment (start 93.3704 92.71) (end 95.2952 94.6348) (width 0.15) (layer "F.Cu") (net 4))
 (segment (start 102.7464 97.2455) (end 109.0257 103.5248) (width 0.15) (layer "B.Cu") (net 18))
 (segment (start 120.4769 110.1494) (end 127.2244 110.1494) (width 0.15) (layer "B.Cu") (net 18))
 (segment (start 102.7464 80.0017) (end 102.7464 97.2455) (width 0.15) (layer "B.Cu") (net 18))
 (segment (start 129.286 108.732) (end 128.1407 108.732) (width 0.15) (layer "B.Cu") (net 18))
 (segment (start 89.46 66.7153) (end 102.7464 80.0017) (width 0.15) (layer "B.Cu") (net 18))
 (segment (start 89.46 65.59) (end 89.46 66.7153) (width 0.15) (layer "B.Cu") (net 18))
 (segment (start 109.0257 103.5248) (end 113.8523 103.5248) (width 0.15) (layer "B.Cu") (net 18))
 (segment (start 127.2244 110.1494) (end 128.1407 109.2331) (width 0.15) (layer "B.Cu") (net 18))
 (segment (start 113.8523 103.5248) (end 120.4769 110.1494) (width 0.15) (layer "B.Cu") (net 18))
 (segment (start 128.1407 109.2331) (end 128.1407 108.732) (width 0.15) (layer "B.Cu") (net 18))
 (segment (start 109.0289 100.9848) (end 118.3546 100.9848) (width 0.15) (layer "B.Cu") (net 17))
 (segment (start 126.746 108.732) (end 125.6007 108.732) (width 0.15) (layer "B.Cu") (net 17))
 (segment (start 125.6007 108.2309) (end 125.6007 108.732) (width 0.15) (layer "B.Cu") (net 17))
 (segment (start 92 66.7153) (end 106.6895 81.4048) (width 0.15) (layer "B.Cu") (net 17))
 (segment (start 106.6895 98.6454) (end 109.0289 100.9848) (width 0.15) (layer "B.Cu") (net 17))
 (segment (start 106.6895 81.4048) (end 106.6895 98.6454) (width 0.15) (layer "B.Cu") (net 17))
 (segment (start 118.3546 100.9848) (end 125.6007 108.2309) (width 0.15) (layer "B.Cu") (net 17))
 (segment (start 92 65.59) (end 92 66.7153) (width 0.15) (layer "B.Cu") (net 17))
 (segment (start 125.9772 79.3974) (end 127.3787 80.7989) (width 0.15) (layer "F.Cu") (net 19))
 (segment (start 100.7453 65.59) (end 100.7453 65.8713) (width 0.15) (layer "F.Cu") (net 19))
 (segment (start 127.3787 80.7989) (end 127.3787 81.3) (width 0.15) (layer "F.Cu") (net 19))
 (segment (start 128.524 81.3) (end 127.3787 81.3) (width 0.15) (layer "F.Cu") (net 19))
 (segment (start 114.2714 79.3974) (end 125.9772 79.3974) (width 0.15) (layer "F.Cu") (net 19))
 (segment (start 99.62 65.59) (end 100.7453 65.59) (width 0.15) (layer "F.Cu") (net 19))
 (segment (start 100.7453 65.8713) (end 114.2714 79.3974) (width 0.15) (layer "F.Cu") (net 19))
 (segment (start 111.8402 66.7153) (end 115.7952 66.7153) (width 0.15) (layer "F.Cu") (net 22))
 (segment (start 110.9053 65.59) (end 110.9053 65.7804) (width 0.15) (layer "F.Cu") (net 22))
 (segment (start 129.413 97.048) (end 129.413 95.6777) (width 0.15) (layer "F.Cu") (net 22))
 (segment (start 109.78 65.59) (end 110.9053 65.59) (width 0.15) (layer "F.Cu") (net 22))
 (segment (start 115.7952 66.7153) (end 129.6745 80.5946) (width 0.15) (layer "F.Cu") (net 22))
 (segment (start 110.9053 65.7804) (end 111.8402 66.7153) (width 0.15) (layer "F.Cu") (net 22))
 (segment (start 129.6745 95.4162) (end 129.413 95.6777) (width 0.15) (layer "F.Cu") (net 22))
 (segment (start 129.6745 80.5946) (end 129.6745 95.4162) (width 0.15) (layer "F.Cu") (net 22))
 (segment (start 113.4453 65.59) (end 113.4453 65.3087) (width 0.15) (layer "B.Cu") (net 21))
 (segment (start 116.13 65.184) (end 116.13 86.305) (width 0.15) (layer "B.Cu") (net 21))
 (segment (start 126.873 97.048) (end 125.7277 97.048) (width 0.15) (layer "B.Cu") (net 21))
 (segment (start 113.4453 65.3087) (end 114.2894 64.4646) (width 0.15) (layer "B.Cu") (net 21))
 (segment (start 114.2894 64.4646) (end 115.4106 64.4646) (width 0.15) (layer "B.Cu") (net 21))
 (segment (start 115.4106 64.4646) (end 116.13 65.184) (width 0.15) (layer "B.Cu") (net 21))
 (segment (start 116.13 86.305) (end 125.7277 95.9027) (width 0.15) (layer "B.Cu") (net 21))
 (segment (start 125.7277 95.9027) (end 125.7277 97.048) (width 0.15) (layer "B.Cu") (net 21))
 (segment (start 112.32 65.59) (end 113.4453 65.59) (width 0.15) (layer "B.Cu") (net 21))
 (segment (start 124.333 95.6777) (end 114.86 86.2047) (width 0.15) (layer "B.Cu") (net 20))
 (segment (start 114.86 86.2047) (end 114.86 65.59) (width 0.15) (layer "B.Cu") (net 20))
 (segment (start 124.333 97.048) (end 124.333 95.6777) (width 0.15) (layer "B.Cu") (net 20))
 (segment (start 122.48 66.7153) (end 131.953 76.1883) (width 0.15) (layer "B.Cu") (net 23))
 (segment (start 122.48 65.59) (end 122.48 66.7153) (width 0.15) (layer "B.Cu") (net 23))
 (segment (start 131.953 76.1883) (end 131.953 97.048) (width 0.15) (layer "B.Cu") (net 23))
 (segment (start 100.1543 100.1562) (end 94.4812 100.1562) (width 0.15) (layer "F.Cu") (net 6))
 (segment (start 101.671 99.7148) (end 100.5957 99.7148) (width 0.15) (layer "F.Cu") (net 6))
 (segment (start 100.5957 99.7148) (end 100.1543 100.1562) (width 0.15) (layer "F.Cu") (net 6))
 (segment (start 94.4812 100.1562) (end 93.385 99.06) (width 0.15) (layer "F.Cu") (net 6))
 (segment (start 96.5798 89.5548) (end 93.385 86.36) (width 0.15) (layer "F.Cu") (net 3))
 (segment (start 101.671 89.5548) (end 96.5798 89.5548) (width 0.15) (layer "F.Cu") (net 3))
 (segment (start 87.5792 100.076) (end 91.7504 95.9048) (width 0.15) (layer "F.Cu") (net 14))
 (segment (start 104.4057 95.9048) (end 108.2157 92.0948) (width 0.15) (layer "F.Cu") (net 14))
 (segment (start 109.291 92.0948) (end 108.2157 92.0948) (width 0.15) (layer "F.Cu") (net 14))
 (segment (start 91.7504 95.9048) (end 104.4057 95.9048) (width 0.15) (layer "F.Cu") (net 14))
 (segment (start 109.1566 98.6395) (end 109.291 98.6395) (width 0.15) (layer "B.Cu") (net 11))
 (segment (start 95.6653 66.5704) (end 107.6902 78.5953) (width 0.15) (layer "B.Cu") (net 11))
 (segment (start 107.6902 97.1731) (end 109.1566 98.6395) (width 0.15) (layer "B.Cu") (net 11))
 (segment (start 95.6653 65.0192) (end 95.6653 66.5704) (width 0.15) (layer "B.Cu") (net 11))
 (segment (start 94.54 63.05) (end 94.54 64.1753) (width 0.15) (layer "B.Cu") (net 11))
 (segment (start 94.8214 64.1753) (end 95.6653 65.0192) (width 0.15) (layer "B.Cu") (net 11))
 (segment (start 94.54 64.1753) (end 94.8214 64.1753) (width 0.15) (layer "B.Cu") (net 11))
 (segment (start 107.6902 78.5953) (end 107.6902 97.1731) (width 0.15) (layer "B.Cu") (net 11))
 (segment (start 109.291 99.7148) (end 109.291 98.6395) (width 0.15) (layer "B.Cu") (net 11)))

